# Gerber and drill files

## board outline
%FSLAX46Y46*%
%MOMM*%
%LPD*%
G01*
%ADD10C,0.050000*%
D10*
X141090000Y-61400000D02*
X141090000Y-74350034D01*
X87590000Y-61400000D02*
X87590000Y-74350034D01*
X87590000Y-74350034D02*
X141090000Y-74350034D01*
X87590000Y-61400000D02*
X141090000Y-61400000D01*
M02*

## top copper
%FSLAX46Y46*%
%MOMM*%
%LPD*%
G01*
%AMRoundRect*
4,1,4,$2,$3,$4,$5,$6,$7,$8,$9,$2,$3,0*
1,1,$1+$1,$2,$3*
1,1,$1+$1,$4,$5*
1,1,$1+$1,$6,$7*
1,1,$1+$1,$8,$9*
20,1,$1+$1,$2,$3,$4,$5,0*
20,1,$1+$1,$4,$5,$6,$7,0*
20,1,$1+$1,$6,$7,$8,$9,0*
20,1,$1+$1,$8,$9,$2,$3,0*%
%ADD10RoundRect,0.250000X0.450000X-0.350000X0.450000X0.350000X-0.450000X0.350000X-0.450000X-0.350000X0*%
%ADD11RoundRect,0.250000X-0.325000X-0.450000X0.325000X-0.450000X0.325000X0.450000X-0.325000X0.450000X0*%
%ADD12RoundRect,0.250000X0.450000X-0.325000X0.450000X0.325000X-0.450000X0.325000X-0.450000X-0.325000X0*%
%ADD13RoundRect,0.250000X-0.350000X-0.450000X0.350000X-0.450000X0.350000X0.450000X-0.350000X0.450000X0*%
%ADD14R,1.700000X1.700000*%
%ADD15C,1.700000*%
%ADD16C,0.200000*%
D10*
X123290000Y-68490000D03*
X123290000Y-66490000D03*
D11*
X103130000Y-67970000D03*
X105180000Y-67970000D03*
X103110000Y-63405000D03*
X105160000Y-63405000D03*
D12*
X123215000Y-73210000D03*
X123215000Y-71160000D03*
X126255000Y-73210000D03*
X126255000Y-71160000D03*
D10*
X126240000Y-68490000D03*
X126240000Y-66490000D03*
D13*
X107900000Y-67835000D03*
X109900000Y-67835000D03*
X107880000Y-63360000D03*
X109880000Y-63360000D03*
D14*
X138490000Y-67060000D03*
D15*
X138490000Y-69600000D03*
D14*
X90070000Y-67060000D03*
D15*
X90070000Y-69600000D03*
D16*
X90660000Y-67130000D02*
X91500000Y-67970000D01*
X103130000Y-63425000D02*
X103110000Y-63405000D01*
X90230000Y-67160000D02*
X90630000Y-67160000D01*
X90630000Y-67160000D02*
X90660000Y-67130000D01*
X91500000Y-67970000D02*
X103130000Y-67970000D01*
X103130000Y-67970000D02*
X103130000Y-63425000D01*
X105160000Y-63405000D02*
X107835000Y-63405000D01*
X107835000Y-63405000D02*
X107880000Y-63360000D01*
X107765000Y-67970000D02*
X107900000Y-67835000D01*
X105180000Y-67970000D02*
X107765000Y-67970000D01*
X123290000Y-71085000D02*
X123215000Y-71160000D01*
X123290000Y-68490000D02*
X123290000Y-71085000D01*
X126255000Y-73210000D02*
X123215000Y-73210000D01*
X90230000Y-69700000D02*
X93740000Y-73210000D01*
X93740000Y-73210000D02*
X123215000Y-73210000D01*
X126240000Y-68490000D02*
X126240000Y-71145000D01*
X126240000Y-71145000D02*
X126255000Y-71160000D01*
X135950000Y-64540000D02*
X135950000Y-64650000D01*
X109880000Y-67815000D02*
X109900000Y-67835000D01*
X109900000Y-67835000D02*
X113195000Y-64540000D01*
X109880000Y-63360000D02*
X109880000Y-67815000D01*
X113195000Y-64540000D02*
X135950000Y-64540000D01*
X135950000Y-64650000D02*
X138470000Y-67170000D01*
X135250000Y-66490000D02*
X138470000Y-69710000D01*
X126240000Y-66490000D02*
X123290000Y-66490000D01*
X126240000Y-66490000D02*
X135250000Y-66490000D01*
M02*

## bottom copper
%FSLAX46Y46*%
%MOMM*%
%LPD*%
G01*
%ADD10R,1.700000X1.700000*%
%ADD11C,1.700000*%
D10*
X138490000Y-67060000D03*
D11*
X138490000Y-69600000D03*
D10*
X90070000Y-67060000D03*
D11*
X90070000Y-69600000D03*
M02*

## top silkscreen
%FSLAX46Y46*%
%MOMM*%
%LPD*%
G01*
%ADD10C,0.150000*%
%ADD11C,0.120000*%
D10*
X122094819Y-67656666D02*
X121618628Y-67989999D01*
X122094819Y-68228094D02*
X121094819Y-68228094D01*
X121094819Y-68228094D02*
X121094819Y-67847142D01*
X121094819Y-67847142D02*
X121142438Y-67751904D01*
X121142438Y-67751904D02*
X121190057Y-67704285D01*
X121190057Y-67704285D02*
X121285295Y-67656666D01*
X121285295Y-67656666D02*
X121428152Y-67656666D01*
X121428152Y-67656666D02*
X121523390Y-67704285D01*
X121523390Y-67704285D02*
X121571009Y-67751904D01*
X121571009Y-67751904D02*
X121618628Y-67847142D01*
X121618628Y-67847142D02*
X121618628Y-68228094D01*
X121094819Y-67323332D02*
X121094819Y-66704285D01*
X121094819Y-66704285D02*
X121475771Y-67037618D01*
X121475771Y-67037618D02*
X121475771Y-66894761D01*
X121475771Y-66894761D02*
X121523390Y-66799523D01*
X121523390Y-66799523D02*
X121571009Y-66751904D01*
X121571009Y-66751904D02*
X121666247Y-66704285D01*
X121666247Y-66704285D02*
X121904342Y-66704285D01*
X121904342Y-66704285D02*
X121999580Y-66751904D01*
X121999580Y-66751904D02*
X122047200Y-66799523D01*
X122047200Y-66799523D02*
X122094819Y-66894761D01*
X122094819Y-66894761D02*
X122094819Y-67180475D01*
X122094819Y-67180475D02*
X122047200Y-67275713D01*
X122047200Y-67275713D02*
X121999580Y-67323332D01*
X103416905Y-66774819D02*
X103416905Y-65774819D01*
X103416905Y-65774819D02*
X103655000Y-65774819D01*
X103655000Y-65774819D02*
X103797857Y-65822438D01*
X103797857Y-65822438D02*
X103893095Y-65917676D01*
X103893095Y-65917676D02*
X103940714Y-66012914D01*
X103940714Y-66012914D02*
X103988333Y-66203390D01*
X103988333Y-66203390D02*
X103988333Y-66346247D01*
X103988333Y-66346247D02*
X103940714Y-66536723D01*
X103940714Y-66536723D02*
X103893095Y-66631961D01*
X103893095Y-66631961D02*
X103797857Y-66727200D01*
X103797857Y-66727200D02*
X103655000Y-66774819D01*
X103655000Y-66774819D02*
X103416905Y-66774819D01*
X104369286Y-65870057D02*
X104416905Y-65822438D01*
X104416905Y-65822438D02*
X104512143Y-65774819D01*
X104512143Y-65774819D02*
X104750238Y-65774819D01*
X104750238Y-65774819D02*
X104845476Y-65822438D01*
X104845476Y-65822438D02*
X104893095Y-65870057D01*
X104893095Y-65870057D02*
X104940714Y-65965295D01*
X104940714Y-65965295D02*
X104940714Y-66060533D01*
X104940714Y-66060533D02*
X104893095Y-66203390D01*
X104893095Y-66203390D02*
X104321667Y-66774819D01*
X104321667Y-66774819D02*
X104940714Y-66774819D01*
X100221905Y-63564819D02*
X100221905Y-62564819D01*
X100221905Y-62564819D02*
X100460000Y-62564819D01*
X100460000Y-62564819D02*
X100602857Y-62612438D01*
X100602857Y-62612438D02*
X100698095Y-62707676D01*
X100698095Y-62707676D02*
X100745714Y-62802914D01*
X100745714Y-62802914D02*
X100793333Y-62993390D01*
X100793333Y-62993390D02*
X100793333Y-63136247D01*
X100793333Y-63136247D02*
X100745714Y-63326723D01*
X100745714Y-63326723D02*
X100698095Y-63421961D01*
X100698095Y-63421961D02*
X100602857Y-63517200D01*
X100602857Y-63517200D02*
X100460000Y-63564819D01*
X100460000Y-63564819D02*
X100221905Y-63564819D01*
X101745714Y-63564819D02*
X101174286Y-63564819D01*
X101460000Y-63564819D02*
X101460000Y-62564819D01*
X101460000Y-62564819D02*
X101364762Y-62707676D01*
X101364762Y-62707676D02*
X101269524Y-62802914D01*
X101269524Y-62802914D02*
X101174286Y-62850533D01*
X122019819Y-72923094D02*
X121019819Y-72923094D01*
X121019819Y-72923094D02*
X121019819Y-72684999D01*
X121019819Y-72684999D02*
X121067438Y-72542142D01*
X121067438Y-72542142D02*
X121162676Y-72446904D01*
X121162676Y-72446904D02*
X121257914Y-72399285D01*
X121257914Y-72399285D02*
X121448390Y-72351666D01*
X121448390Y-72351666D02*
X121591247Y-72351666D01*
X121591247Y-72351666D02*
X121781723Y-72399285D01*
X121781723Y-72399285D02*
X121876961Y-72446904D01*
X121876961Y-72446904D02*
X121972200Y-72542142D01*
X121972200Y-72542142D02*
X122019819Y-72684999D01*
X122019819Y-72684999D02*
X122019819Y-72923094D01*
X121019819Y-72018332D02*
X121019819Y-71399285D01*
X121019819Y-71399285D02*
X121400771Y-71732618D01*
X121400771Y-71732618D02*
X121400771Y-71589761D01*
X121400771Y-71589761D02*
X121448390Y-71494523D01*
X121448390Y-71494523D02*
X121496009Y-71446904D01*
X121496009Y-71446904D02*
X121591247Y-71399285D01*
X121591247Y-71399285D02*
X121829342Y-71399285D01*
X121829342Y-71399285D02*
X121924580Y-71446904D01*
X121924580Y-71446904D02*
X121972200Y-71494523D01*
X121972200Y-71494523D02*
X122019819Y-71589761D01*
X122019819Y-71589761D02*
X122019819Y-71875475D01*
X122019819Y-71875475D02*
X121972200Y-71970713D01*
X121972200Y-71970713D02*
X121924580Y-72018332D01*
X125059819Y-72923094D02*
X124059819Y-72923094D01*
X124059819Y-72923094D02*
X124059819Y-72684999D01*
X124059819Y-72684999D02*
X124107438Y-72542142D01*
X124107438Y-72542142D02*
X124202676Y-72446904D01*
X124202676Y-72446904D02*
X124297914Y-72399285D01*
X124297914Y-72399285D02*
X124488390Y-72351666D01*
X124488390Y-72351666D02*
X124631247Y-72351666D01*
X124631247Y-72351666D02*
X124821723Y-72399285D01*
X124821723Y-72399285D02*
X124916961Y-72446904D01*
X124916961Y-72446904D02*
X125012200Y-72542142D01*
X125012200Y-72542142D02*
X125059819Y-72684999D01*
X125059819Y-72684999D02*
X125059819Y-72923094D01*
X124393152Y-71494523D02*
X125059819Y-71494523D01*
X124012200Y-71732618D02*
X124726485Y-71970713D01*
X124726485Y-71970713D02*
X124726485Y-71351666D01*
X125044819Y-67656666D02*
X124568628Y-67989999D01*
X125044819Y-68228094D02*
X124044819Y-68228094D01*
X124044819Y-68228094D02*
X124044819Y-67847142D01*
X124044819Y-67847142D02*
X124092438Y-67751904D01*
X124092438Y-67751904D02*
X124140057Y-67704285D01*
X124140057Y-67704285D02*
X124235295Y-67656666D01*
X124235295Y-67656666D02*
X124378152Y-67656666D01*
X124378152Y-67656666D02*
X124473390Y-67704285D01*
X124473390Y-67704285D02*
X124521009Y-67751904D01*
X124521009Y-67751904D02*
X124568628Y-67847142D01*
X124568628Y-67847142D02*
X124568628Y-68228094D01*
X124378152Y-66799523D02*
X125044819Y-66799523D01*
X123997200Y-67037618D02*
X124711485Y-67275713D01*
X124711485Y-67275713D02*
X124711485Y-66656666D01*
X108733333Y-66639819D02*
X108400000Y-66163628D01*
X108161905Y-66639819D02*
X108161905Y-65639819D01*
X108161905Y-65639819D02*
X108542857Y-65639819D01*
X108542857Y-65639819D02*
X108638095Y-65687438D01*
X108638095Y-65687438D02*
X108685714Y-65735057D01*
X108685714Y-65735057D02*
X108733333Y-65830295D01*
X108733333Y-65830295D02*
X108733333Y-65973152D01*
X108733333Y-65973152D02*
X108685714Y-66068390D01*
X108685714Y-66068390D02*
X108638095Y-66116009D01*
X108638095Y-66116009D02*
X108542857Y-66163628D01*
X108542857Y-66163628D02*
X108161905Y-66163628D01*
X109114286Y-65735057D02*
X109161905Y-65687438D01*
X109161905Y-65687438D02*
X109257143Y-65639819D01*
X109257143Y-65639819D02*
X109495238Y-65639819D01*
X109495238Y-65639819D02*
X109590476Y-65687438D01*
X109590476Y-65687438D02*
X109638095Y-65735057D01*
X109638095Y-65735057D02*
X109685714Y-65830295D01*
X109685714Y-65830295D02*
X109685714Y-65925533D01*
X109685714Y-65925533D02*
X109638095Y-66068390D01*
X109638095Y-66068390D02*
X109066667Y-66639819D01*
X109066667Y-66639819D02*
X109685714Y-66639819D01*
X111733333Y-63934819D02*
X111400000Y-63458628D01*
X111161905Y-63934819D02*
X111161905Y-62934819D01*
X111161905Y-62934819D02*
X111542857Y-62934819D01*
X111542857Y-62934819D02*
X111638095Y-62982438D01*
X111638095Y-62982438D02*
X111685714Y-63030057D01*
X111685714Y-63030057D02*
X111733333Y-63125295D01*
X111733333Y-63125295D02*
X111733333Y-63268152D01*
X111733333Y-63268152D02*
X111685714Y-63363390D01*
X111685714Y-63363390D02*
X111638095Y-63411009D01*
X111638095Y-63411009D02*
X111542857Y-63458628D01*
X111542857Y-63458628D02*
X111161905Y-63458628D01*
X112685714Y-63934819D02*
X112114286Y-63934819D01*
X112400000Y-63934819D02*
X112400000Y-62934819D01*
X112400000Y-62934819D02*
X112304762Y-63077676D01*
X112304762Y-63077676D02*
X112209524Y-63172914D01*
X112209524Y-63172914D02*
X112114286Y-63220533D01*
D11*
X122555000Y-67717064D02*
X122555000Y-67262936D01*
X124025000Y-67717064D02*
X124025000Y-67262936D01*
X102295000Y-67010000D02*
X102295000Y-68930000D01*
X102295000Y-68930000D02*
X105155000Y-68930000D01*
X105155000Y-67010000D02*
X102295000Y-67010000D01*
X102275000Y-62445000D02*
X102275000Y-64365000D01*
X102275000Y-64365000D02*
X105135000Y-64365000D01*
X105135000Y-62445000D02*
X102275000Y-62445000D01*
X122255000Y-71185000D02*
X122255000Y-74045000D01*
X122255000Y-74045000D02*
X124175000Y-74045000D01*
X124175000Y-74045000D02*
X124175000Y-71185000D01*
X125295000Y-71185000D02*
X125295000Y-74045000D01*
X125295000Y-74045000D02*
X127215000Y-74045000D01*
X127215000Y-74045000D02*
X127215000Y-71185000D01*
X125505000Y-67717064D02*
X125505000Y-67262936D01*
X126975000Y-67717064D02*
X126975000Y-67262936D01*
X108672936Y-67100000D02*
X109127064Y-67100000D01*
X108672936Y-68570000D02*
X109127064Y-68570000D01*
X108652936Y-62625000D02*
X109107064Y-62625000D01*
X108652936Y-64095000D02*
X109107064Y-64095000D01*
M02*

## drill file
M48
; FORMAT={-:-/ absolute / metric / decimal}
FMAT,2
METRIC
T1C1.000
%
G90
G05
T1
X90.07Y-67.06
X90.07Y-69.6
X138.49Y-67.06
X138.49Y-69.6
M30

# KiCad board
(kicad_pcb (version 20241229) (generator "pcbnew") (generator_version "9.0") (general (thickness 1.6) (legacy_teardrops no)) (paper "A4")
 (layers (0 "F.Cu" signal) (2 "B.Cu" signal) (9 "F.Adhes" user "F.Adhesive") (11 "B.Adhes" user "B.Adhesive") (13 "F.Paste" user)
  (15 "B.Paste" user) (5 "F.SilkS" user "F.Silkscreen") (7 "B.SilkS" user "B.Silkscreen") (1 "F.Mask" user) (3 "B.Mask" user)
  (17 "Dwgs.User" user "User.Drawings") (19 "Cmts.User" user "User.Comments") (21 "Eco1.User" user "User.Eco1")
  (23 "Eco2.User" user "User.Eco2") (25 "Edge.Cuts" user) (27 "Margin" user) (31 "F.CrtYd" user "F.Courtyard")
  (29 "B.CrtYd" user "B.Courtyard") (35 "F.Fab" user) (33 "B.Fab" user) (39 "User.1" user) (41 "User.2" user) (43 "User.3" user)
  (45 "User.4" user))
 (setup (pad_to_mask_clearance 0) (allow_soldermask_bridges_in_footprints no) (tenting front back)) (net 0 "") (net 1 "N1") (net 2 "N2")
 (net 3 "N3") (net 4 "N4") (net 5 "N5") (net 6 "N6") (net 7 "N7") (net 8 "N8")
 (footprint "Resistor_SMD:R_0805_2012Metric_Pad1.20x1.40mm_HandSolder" (layer "F.Cu") (at 123.29 67.49 90)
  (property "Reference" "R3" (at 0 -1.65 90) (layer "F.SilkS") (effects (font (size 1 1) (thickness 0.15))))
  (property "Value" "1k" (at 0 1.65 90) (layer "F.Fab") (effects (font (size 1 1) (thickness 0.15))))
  (fp_line (start -0.227064 -0.735) (end 0.227064 -0.735) (stroke (width 0.12) (type solid)) (layer "F.SilkS"))
  (fp_line (start -0.227064 0.735) (end 0.227064 0.735) (stroke (width 0.12) (type solid)) (layer "F.SilkS"))
  (pad "1" smd roundrect (at -1 0 90) (size 1.2 1.4) (layers "F.Cu" "F.Mask" "F.Paste") (roundrect_rratio 0.208333) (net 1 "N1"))
  (pad "2" smd roundrect (at 1 0 90) (size 1.2 1.4) (layers "F.Cu" "F.Mask" "F.Paste") (roundrect_rratio 0.208333) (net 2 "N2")))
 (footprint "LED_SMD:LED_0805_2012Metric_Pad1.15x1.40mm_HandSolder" (layer "F.Cu") (at 104.155 67.97)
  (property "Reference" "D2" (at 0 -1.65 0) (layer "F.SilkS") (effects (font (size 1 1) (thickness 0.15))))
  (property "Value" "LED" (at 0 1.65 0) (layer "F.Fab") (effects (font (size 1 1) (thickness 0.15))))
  (fp_line (start -1.86 -0.96) (end -1.86 0.96) (stroke (width 0.12) (type solid)) (layer "F.SilkS"))
  (fp_line (start -1.86 0.96) (end 1 0.96) (stroke (width 0.12) (type solid)) (layer "F.SilkS"))
  (fp_line (start 1 -0.96) (end -1.86 -0.96) (stroke (width 0.12) (type solid)) (layer "F.SilkS"))
  (pad "1" smd roundrect (at -1.025 0) (size 1.15 1.4) (layers "F.Cu" "F.Mask" "F.Paste") (roundrect_rratio 0.217391) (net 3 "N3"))
  (pad "2" smd roundrect (at 1.025 0) (size 1.15 1.4) (layers "F.Cu" "F.Mask" "F.Paste") (roundrect_rratio 0.217391) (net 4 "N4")))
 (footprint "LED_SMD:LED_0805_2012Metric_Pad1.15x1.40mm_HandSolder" (layer "F.Cu") (at 104.135 63.405)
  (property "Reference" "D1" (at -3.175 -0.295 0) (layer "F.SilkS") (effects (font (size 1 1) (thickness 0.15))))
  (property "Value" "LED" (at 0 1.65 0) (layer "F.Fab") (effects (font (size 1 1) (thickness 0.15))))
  (fp_line (start -1.86 -0.96) (end -1.86 0.96) (stroke (width 0.12) (type solid)) (layer "F.SilkS"))
  (fp_line (start -1.86 0.96) (end 1 0.96) (stroke (width 0.12) (type solid)) (layer "F.SilkS"))
  (fp_line (start 1 -0.96) (end -1.86 -0.96) (stroke (width 0.12) (type solid)) (layer "F.SilkS"))
  (pad "1" smd roundrect (at -1.025 0) (size 1.15 1.4) (layers "F.Cu" "F.Mask" "F.Paste") (roundrect_rratio 0.217391) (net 3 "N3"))
  (pad "2" smd roundrect (at 1.025 0) (size 1.15 1.4) (layers "F.Cu" "F.Mask" "F.Paste") (roundrect_rratio 0.217391) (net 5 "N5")))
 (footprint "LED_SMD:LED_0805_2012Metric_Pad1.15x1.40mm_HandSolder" (layer "F.Cu") (at 123.215 72.185 90)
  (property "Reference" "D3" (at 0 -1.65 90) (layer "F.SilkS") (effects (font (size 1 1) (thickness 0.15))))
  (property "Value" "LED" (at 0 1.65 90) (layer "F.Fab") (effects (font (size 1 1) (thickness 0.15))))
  (fp_line (start 1 -0.96) (end -1.86 -0.96) (stroke (width 0.12) (type solid)) (layer "F.SilkS"))
  (fp_line (start -1.86 -0.96) (end -1.86 0.96) (stroke (width 0.12) (type solid)) (layer "F.SilkS"))
  (fp_line (start -1.86 0.96) (end 1 0.96) (stroke (width 0.12) (type solid)) (layer "F.SilkS"))
  (pad "1" smd roundrect (at -1.025 0 90) (size 1.15 1.4) (layers "F.Cu" "F.Mask" "F.Paste") (roundrect_rratio 0.217391) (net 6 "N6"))
  (pad "2" smd roundrect (at 1.025 0 90) (size 1.15 1.4) (layers "F.Cu" "F.Mask" "F.Paste") (roundrect_rratio 0.217391) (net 1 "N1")))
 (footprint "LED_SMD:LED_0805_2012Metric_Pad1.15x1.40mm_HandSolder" (layer "F.Cu") (at 126.255 72.185 90)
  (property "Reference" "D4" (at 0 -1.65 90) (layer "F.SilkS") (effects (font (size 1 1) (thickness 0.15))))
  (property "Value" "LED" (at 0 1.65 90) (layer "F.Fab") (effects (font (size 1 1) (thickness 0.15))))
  (fp_line (start 1 -0.96) (end -1.86 -0.96) (stroke (width 0.12) (type solid)) (layer "F.SilkS"))
  (fp_line (start -1.86 -0.96) (end -1.86 0.96) (stroke (width 0.12) (type solid)) (layer "F.SilkS"))
  (fp_line (start -1.86 0.96) (end 1 0.96) (stroke (width 0.12) (type solid)) (layer "F.SilkS"))
  (pad "1" smd roundrect (at -1.025 0 90) (size 1.15 1.4) (layers "F.Cu" "F.Mask" "F.Paste") (roundrect_rratio 0.217391) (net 6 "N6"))
  (pad "2" smd roundrect (at 1.025 0 90) (size 1.15 1.4) (layers "F.Cu" "F.Mask" "F.Paste") (roundrect_rratio 0.217391) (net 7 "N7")))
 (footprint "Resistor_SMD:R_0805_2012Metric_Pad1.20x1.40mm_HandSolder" (layer "F.Cu") (at 126.24 67.49 90)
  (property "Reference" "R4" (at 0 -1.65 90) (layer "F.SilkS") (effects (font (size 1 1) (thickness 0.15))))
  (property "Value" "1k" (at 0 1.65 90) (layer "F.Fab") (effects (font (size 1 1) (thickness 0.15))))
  (fp_line (start -0.227064 -0.735) (end 0.227064 -0.735) (stroke (width 0.12) (type solid)) (layer "F.SilkS"))
  (fp_line (start -0.227064 0.735) (end 0.227064 0.735) (stroke (width 0.12) (type solid)) (layer "F.SilkS"))
  (pad "1" smd roundrect (at -1 0 90) (size 1.2 1.4) (layers "F.Cu" "F.Mask" "F.Paste") (roundrect_rratio 0.208333) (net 7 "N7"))
  (pad "2" smd roundrect (at 1 0 90) (size 1.2 1.4) (layers "F.Cu" "F.Mask" "F.Paste") (roundrect_rratio 0.208333) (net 2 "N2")))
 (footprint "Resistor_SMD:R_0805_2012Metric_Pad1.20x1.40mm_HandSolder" (layer "F.Cu") (at 108.9 67.835)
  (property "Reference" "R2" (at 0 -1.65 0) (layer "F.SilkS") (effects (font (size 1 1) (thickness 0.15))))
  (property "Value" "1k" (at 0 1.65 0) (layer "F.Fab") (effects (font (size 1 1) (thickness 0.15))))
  (fp_line (start -0.227064 -0.735) (end 0.227064 -0.735) (stroke (width 0.12) (type solid)) (layer "F.SilkS"))
  (fp_line (start -0.227064 0.735) (end 0.227064 0.735) (stroke (width 0.12) (type solid)) (layer "F.SilkS"))
  (pad "1" smd roundrect (at -1 0) (size 1.2 1.4) (layers "F.Cu" "F.Mask" "F.Paste") (roundrect_rratio 0.208333) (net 4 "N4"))
  (pad "2" smd roundrect (at 1 0) (size 1.2 1.4) (layers "F.Cu" "F.Mask" "F.Paste") (roundrect_rratio 0.208333) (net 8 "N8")))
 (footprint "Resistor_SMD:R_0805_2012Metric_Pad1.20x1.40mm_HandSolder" (layer "F.Cu") (at 108.88 63.36)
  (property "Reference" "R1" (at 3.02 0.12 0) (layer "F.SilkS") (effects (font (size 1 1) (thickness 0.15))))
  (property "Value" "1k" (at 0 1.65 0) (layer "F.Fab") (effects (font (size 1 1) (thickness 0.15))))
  (fp_line (start -0.227064 -0.735) (end 0.227064 -0.735) (stroke (width 0.12) (type solid)) (layer "F.SilkS"))
  (fp_line (start -0.227064 0.735) (end 0.227064 0.735) (stroke (width 0.12) (type solid)) (layer "F.SilkS"))
  (pad "1" smd roundrect (at -1 0) (size 1.2 1.4) (layers "F.Cu" "F.Mask" "F.Paste") (roundrect_rratio 0.208333) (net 5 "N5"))
  (pad "2" smd roundrect (at 1 0) (size 1.2 1.4) (layers "F.Cu" "F.Mask" "F.Paste") (roundrect_rratio 0.208333) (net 8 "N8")))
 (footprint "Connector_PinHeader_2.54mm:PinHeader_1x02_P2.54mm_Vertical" (layer "B.Cu") (at 138.49 67.06 180)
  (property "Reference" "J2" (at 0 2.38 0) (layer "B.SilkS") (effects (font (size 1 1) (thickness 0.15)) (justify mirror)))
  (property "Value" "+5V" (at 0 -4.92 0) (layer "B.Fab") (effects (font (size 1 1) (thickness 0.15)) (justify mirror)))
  (pad "1" thru_hole rect (at 0 0 180) (size 1.7 1.7) (drill 1) (layers "*.Cu" "*.Mask") (remove_unused_layers no) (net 2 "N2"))
  (pad "2" thru_hole circle (at 0 -2.54 180) (size 1.7 1.7) (drill 1) (layers "*.Cu" "*.Mask") (remove_unused_layers no) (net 8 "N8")))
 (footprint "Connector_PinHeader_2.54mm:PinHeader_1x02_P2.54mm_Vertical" (layer "B.Cu") (at 90.07 67.06 180)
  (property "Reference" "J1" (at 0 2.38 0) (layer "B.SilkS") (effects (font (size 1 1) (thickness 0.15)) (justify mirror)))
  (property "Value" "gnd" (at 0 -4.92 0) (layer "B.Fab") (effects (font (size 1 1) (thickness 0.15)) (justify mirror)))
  (pad "1" thru_hole rect (at 0 0 180) (size 1.7 1.7) (drill 1) (layers "*.Cu" "*.Mask") (remove_unused_layers no) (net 3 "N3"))
  (pad "2" thru_hole circle (at 0 -2.54 180) (size 1.7 1.7) (drill 1) (layers "*.Cu" "*.Mask") (remove_unused_layers no) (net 6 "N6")))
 (gr_line (start 141.09 61.4) (end 141.09 74.350034) (stroke (width 0.05) (type solid)) (layer "Edge.Cuts"))
 (gr_line (start 87.59 61.4) (end 87.59 74.350034) (stroke (width 0.05) (type solid)) (layer "Edge.Cuts"))
 (gr_line (start 87.59 74.350034) (end 141.09 74.350034) (stroke (width 0.05) (type solid)) (layer "Edge.Cuts"))
 (gr_line (start 87.59 61.4) (end 141.09 61.4) (stroke (width 0.05) (type solid)) (layer "Edge.Cuts"))
 (segment (start 90.66 67.13) (end 91.5 67.97) (width 0.2) (layer "F.Cu") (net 3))
 (segment (start 103.13 63.425) (end 103.11 63.405) (width 0.2) (layer "F.Cu") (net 3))
 (segment (start 90.23 67.16) (end 90.63 67.16) (width 0.2) (layer "F.Cu") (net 3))
 (segment (start 90.63 67.16) (end 90.66 67.13) (width 0.2) (layer "F.Cu") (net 3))
 (segment (start 91.5 67.97) (end 103.13 67.97) (width 0.2) (layer "F.Cu") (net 3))
 (segment (start 103.13 67.97) (end 103.13 63.425) (width 0.2) (layer "F.Cu") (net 3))
 (segment (start 105.16 63.405) (end 107.835 63.405) (width 0.2) (layer "F.Cu") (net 5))
 (segment (start 107.835 63.405) (end 107.88 63.36) (width 0.2) (layer "F.Cu") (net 5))
 (segment (start 107.765 67.97) (end 107.9 67.835) (width 0.2) (layer "F.Cu") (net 4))
 (segment (start 105.18 67.97) (end 107.765 67.97) (width 0.2) (layer "F.Cu") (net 4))
 (segment (start 123.29 71.085) (end 123.215 71.16) (width 0.2) (layer "F.Cu") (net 1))
 (segment (start 123.29 68.49) (end 123.29 71.085) (width 0.2) (layer "F.Cu") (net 1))
 (segment (start 126.255 73.21) (end 123.215 73.21) (width 0.2) (layer "F.Cu") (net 6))
 (segment (start 90.23 69.7) (end 93.74 73.21) (width 0.2) (layer "F.Cu") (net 6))
 (segment (start 93.74 73.21) (end 123.215 73.21) (width 0.2) (layer "F.Cu") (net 6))
 (segment (start 126.24 68.49) (end 126.24 71.145) (width 0.2) (layer "F.Cu") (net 7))
 (segment (start 126.24 71.145) (end 126.255 71.16) (width 0.2) (layer "F.Cu") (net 7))
 (segment (start 135.95 64.54) (end 135.95 64.65) (width 0.2) (layer "F.Cu") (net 8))
 (segment (start 109.88 67.815) (end 109.9 67.835) (width 0.2) (layer "F.Cu") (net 8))
 (segment (start 109.9 67.835) (end 113.195 64.54) (width 0.2) (layer "F.Cu") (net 8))
 (segment (start 109.88 63.36) (end 109.88 67.815) (width 0.2) (layer "F.Cu") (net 8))
 (segment (start 113.195 64.54) (end 135.95 64.54) (width 0.2) (layer "F.Cu") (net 8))
 (segment (start 135.95 64.65) (end 138.47 67.17) (width 0.2) (layer "F.Cu") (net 8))
 (segment (start 135.25 66.49) (end 138.47 69.71) (width 0.2) (layer "F.Cu") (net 2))
 (segment (start 126.24 66.49) (end 123.29 66.49) (width 0.2) (layer "F.Cu") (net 2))
 (segment (start 126.24 66.49) (end 135.25 66.49) (width 0.2) (layer "F.Cu") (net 2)))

